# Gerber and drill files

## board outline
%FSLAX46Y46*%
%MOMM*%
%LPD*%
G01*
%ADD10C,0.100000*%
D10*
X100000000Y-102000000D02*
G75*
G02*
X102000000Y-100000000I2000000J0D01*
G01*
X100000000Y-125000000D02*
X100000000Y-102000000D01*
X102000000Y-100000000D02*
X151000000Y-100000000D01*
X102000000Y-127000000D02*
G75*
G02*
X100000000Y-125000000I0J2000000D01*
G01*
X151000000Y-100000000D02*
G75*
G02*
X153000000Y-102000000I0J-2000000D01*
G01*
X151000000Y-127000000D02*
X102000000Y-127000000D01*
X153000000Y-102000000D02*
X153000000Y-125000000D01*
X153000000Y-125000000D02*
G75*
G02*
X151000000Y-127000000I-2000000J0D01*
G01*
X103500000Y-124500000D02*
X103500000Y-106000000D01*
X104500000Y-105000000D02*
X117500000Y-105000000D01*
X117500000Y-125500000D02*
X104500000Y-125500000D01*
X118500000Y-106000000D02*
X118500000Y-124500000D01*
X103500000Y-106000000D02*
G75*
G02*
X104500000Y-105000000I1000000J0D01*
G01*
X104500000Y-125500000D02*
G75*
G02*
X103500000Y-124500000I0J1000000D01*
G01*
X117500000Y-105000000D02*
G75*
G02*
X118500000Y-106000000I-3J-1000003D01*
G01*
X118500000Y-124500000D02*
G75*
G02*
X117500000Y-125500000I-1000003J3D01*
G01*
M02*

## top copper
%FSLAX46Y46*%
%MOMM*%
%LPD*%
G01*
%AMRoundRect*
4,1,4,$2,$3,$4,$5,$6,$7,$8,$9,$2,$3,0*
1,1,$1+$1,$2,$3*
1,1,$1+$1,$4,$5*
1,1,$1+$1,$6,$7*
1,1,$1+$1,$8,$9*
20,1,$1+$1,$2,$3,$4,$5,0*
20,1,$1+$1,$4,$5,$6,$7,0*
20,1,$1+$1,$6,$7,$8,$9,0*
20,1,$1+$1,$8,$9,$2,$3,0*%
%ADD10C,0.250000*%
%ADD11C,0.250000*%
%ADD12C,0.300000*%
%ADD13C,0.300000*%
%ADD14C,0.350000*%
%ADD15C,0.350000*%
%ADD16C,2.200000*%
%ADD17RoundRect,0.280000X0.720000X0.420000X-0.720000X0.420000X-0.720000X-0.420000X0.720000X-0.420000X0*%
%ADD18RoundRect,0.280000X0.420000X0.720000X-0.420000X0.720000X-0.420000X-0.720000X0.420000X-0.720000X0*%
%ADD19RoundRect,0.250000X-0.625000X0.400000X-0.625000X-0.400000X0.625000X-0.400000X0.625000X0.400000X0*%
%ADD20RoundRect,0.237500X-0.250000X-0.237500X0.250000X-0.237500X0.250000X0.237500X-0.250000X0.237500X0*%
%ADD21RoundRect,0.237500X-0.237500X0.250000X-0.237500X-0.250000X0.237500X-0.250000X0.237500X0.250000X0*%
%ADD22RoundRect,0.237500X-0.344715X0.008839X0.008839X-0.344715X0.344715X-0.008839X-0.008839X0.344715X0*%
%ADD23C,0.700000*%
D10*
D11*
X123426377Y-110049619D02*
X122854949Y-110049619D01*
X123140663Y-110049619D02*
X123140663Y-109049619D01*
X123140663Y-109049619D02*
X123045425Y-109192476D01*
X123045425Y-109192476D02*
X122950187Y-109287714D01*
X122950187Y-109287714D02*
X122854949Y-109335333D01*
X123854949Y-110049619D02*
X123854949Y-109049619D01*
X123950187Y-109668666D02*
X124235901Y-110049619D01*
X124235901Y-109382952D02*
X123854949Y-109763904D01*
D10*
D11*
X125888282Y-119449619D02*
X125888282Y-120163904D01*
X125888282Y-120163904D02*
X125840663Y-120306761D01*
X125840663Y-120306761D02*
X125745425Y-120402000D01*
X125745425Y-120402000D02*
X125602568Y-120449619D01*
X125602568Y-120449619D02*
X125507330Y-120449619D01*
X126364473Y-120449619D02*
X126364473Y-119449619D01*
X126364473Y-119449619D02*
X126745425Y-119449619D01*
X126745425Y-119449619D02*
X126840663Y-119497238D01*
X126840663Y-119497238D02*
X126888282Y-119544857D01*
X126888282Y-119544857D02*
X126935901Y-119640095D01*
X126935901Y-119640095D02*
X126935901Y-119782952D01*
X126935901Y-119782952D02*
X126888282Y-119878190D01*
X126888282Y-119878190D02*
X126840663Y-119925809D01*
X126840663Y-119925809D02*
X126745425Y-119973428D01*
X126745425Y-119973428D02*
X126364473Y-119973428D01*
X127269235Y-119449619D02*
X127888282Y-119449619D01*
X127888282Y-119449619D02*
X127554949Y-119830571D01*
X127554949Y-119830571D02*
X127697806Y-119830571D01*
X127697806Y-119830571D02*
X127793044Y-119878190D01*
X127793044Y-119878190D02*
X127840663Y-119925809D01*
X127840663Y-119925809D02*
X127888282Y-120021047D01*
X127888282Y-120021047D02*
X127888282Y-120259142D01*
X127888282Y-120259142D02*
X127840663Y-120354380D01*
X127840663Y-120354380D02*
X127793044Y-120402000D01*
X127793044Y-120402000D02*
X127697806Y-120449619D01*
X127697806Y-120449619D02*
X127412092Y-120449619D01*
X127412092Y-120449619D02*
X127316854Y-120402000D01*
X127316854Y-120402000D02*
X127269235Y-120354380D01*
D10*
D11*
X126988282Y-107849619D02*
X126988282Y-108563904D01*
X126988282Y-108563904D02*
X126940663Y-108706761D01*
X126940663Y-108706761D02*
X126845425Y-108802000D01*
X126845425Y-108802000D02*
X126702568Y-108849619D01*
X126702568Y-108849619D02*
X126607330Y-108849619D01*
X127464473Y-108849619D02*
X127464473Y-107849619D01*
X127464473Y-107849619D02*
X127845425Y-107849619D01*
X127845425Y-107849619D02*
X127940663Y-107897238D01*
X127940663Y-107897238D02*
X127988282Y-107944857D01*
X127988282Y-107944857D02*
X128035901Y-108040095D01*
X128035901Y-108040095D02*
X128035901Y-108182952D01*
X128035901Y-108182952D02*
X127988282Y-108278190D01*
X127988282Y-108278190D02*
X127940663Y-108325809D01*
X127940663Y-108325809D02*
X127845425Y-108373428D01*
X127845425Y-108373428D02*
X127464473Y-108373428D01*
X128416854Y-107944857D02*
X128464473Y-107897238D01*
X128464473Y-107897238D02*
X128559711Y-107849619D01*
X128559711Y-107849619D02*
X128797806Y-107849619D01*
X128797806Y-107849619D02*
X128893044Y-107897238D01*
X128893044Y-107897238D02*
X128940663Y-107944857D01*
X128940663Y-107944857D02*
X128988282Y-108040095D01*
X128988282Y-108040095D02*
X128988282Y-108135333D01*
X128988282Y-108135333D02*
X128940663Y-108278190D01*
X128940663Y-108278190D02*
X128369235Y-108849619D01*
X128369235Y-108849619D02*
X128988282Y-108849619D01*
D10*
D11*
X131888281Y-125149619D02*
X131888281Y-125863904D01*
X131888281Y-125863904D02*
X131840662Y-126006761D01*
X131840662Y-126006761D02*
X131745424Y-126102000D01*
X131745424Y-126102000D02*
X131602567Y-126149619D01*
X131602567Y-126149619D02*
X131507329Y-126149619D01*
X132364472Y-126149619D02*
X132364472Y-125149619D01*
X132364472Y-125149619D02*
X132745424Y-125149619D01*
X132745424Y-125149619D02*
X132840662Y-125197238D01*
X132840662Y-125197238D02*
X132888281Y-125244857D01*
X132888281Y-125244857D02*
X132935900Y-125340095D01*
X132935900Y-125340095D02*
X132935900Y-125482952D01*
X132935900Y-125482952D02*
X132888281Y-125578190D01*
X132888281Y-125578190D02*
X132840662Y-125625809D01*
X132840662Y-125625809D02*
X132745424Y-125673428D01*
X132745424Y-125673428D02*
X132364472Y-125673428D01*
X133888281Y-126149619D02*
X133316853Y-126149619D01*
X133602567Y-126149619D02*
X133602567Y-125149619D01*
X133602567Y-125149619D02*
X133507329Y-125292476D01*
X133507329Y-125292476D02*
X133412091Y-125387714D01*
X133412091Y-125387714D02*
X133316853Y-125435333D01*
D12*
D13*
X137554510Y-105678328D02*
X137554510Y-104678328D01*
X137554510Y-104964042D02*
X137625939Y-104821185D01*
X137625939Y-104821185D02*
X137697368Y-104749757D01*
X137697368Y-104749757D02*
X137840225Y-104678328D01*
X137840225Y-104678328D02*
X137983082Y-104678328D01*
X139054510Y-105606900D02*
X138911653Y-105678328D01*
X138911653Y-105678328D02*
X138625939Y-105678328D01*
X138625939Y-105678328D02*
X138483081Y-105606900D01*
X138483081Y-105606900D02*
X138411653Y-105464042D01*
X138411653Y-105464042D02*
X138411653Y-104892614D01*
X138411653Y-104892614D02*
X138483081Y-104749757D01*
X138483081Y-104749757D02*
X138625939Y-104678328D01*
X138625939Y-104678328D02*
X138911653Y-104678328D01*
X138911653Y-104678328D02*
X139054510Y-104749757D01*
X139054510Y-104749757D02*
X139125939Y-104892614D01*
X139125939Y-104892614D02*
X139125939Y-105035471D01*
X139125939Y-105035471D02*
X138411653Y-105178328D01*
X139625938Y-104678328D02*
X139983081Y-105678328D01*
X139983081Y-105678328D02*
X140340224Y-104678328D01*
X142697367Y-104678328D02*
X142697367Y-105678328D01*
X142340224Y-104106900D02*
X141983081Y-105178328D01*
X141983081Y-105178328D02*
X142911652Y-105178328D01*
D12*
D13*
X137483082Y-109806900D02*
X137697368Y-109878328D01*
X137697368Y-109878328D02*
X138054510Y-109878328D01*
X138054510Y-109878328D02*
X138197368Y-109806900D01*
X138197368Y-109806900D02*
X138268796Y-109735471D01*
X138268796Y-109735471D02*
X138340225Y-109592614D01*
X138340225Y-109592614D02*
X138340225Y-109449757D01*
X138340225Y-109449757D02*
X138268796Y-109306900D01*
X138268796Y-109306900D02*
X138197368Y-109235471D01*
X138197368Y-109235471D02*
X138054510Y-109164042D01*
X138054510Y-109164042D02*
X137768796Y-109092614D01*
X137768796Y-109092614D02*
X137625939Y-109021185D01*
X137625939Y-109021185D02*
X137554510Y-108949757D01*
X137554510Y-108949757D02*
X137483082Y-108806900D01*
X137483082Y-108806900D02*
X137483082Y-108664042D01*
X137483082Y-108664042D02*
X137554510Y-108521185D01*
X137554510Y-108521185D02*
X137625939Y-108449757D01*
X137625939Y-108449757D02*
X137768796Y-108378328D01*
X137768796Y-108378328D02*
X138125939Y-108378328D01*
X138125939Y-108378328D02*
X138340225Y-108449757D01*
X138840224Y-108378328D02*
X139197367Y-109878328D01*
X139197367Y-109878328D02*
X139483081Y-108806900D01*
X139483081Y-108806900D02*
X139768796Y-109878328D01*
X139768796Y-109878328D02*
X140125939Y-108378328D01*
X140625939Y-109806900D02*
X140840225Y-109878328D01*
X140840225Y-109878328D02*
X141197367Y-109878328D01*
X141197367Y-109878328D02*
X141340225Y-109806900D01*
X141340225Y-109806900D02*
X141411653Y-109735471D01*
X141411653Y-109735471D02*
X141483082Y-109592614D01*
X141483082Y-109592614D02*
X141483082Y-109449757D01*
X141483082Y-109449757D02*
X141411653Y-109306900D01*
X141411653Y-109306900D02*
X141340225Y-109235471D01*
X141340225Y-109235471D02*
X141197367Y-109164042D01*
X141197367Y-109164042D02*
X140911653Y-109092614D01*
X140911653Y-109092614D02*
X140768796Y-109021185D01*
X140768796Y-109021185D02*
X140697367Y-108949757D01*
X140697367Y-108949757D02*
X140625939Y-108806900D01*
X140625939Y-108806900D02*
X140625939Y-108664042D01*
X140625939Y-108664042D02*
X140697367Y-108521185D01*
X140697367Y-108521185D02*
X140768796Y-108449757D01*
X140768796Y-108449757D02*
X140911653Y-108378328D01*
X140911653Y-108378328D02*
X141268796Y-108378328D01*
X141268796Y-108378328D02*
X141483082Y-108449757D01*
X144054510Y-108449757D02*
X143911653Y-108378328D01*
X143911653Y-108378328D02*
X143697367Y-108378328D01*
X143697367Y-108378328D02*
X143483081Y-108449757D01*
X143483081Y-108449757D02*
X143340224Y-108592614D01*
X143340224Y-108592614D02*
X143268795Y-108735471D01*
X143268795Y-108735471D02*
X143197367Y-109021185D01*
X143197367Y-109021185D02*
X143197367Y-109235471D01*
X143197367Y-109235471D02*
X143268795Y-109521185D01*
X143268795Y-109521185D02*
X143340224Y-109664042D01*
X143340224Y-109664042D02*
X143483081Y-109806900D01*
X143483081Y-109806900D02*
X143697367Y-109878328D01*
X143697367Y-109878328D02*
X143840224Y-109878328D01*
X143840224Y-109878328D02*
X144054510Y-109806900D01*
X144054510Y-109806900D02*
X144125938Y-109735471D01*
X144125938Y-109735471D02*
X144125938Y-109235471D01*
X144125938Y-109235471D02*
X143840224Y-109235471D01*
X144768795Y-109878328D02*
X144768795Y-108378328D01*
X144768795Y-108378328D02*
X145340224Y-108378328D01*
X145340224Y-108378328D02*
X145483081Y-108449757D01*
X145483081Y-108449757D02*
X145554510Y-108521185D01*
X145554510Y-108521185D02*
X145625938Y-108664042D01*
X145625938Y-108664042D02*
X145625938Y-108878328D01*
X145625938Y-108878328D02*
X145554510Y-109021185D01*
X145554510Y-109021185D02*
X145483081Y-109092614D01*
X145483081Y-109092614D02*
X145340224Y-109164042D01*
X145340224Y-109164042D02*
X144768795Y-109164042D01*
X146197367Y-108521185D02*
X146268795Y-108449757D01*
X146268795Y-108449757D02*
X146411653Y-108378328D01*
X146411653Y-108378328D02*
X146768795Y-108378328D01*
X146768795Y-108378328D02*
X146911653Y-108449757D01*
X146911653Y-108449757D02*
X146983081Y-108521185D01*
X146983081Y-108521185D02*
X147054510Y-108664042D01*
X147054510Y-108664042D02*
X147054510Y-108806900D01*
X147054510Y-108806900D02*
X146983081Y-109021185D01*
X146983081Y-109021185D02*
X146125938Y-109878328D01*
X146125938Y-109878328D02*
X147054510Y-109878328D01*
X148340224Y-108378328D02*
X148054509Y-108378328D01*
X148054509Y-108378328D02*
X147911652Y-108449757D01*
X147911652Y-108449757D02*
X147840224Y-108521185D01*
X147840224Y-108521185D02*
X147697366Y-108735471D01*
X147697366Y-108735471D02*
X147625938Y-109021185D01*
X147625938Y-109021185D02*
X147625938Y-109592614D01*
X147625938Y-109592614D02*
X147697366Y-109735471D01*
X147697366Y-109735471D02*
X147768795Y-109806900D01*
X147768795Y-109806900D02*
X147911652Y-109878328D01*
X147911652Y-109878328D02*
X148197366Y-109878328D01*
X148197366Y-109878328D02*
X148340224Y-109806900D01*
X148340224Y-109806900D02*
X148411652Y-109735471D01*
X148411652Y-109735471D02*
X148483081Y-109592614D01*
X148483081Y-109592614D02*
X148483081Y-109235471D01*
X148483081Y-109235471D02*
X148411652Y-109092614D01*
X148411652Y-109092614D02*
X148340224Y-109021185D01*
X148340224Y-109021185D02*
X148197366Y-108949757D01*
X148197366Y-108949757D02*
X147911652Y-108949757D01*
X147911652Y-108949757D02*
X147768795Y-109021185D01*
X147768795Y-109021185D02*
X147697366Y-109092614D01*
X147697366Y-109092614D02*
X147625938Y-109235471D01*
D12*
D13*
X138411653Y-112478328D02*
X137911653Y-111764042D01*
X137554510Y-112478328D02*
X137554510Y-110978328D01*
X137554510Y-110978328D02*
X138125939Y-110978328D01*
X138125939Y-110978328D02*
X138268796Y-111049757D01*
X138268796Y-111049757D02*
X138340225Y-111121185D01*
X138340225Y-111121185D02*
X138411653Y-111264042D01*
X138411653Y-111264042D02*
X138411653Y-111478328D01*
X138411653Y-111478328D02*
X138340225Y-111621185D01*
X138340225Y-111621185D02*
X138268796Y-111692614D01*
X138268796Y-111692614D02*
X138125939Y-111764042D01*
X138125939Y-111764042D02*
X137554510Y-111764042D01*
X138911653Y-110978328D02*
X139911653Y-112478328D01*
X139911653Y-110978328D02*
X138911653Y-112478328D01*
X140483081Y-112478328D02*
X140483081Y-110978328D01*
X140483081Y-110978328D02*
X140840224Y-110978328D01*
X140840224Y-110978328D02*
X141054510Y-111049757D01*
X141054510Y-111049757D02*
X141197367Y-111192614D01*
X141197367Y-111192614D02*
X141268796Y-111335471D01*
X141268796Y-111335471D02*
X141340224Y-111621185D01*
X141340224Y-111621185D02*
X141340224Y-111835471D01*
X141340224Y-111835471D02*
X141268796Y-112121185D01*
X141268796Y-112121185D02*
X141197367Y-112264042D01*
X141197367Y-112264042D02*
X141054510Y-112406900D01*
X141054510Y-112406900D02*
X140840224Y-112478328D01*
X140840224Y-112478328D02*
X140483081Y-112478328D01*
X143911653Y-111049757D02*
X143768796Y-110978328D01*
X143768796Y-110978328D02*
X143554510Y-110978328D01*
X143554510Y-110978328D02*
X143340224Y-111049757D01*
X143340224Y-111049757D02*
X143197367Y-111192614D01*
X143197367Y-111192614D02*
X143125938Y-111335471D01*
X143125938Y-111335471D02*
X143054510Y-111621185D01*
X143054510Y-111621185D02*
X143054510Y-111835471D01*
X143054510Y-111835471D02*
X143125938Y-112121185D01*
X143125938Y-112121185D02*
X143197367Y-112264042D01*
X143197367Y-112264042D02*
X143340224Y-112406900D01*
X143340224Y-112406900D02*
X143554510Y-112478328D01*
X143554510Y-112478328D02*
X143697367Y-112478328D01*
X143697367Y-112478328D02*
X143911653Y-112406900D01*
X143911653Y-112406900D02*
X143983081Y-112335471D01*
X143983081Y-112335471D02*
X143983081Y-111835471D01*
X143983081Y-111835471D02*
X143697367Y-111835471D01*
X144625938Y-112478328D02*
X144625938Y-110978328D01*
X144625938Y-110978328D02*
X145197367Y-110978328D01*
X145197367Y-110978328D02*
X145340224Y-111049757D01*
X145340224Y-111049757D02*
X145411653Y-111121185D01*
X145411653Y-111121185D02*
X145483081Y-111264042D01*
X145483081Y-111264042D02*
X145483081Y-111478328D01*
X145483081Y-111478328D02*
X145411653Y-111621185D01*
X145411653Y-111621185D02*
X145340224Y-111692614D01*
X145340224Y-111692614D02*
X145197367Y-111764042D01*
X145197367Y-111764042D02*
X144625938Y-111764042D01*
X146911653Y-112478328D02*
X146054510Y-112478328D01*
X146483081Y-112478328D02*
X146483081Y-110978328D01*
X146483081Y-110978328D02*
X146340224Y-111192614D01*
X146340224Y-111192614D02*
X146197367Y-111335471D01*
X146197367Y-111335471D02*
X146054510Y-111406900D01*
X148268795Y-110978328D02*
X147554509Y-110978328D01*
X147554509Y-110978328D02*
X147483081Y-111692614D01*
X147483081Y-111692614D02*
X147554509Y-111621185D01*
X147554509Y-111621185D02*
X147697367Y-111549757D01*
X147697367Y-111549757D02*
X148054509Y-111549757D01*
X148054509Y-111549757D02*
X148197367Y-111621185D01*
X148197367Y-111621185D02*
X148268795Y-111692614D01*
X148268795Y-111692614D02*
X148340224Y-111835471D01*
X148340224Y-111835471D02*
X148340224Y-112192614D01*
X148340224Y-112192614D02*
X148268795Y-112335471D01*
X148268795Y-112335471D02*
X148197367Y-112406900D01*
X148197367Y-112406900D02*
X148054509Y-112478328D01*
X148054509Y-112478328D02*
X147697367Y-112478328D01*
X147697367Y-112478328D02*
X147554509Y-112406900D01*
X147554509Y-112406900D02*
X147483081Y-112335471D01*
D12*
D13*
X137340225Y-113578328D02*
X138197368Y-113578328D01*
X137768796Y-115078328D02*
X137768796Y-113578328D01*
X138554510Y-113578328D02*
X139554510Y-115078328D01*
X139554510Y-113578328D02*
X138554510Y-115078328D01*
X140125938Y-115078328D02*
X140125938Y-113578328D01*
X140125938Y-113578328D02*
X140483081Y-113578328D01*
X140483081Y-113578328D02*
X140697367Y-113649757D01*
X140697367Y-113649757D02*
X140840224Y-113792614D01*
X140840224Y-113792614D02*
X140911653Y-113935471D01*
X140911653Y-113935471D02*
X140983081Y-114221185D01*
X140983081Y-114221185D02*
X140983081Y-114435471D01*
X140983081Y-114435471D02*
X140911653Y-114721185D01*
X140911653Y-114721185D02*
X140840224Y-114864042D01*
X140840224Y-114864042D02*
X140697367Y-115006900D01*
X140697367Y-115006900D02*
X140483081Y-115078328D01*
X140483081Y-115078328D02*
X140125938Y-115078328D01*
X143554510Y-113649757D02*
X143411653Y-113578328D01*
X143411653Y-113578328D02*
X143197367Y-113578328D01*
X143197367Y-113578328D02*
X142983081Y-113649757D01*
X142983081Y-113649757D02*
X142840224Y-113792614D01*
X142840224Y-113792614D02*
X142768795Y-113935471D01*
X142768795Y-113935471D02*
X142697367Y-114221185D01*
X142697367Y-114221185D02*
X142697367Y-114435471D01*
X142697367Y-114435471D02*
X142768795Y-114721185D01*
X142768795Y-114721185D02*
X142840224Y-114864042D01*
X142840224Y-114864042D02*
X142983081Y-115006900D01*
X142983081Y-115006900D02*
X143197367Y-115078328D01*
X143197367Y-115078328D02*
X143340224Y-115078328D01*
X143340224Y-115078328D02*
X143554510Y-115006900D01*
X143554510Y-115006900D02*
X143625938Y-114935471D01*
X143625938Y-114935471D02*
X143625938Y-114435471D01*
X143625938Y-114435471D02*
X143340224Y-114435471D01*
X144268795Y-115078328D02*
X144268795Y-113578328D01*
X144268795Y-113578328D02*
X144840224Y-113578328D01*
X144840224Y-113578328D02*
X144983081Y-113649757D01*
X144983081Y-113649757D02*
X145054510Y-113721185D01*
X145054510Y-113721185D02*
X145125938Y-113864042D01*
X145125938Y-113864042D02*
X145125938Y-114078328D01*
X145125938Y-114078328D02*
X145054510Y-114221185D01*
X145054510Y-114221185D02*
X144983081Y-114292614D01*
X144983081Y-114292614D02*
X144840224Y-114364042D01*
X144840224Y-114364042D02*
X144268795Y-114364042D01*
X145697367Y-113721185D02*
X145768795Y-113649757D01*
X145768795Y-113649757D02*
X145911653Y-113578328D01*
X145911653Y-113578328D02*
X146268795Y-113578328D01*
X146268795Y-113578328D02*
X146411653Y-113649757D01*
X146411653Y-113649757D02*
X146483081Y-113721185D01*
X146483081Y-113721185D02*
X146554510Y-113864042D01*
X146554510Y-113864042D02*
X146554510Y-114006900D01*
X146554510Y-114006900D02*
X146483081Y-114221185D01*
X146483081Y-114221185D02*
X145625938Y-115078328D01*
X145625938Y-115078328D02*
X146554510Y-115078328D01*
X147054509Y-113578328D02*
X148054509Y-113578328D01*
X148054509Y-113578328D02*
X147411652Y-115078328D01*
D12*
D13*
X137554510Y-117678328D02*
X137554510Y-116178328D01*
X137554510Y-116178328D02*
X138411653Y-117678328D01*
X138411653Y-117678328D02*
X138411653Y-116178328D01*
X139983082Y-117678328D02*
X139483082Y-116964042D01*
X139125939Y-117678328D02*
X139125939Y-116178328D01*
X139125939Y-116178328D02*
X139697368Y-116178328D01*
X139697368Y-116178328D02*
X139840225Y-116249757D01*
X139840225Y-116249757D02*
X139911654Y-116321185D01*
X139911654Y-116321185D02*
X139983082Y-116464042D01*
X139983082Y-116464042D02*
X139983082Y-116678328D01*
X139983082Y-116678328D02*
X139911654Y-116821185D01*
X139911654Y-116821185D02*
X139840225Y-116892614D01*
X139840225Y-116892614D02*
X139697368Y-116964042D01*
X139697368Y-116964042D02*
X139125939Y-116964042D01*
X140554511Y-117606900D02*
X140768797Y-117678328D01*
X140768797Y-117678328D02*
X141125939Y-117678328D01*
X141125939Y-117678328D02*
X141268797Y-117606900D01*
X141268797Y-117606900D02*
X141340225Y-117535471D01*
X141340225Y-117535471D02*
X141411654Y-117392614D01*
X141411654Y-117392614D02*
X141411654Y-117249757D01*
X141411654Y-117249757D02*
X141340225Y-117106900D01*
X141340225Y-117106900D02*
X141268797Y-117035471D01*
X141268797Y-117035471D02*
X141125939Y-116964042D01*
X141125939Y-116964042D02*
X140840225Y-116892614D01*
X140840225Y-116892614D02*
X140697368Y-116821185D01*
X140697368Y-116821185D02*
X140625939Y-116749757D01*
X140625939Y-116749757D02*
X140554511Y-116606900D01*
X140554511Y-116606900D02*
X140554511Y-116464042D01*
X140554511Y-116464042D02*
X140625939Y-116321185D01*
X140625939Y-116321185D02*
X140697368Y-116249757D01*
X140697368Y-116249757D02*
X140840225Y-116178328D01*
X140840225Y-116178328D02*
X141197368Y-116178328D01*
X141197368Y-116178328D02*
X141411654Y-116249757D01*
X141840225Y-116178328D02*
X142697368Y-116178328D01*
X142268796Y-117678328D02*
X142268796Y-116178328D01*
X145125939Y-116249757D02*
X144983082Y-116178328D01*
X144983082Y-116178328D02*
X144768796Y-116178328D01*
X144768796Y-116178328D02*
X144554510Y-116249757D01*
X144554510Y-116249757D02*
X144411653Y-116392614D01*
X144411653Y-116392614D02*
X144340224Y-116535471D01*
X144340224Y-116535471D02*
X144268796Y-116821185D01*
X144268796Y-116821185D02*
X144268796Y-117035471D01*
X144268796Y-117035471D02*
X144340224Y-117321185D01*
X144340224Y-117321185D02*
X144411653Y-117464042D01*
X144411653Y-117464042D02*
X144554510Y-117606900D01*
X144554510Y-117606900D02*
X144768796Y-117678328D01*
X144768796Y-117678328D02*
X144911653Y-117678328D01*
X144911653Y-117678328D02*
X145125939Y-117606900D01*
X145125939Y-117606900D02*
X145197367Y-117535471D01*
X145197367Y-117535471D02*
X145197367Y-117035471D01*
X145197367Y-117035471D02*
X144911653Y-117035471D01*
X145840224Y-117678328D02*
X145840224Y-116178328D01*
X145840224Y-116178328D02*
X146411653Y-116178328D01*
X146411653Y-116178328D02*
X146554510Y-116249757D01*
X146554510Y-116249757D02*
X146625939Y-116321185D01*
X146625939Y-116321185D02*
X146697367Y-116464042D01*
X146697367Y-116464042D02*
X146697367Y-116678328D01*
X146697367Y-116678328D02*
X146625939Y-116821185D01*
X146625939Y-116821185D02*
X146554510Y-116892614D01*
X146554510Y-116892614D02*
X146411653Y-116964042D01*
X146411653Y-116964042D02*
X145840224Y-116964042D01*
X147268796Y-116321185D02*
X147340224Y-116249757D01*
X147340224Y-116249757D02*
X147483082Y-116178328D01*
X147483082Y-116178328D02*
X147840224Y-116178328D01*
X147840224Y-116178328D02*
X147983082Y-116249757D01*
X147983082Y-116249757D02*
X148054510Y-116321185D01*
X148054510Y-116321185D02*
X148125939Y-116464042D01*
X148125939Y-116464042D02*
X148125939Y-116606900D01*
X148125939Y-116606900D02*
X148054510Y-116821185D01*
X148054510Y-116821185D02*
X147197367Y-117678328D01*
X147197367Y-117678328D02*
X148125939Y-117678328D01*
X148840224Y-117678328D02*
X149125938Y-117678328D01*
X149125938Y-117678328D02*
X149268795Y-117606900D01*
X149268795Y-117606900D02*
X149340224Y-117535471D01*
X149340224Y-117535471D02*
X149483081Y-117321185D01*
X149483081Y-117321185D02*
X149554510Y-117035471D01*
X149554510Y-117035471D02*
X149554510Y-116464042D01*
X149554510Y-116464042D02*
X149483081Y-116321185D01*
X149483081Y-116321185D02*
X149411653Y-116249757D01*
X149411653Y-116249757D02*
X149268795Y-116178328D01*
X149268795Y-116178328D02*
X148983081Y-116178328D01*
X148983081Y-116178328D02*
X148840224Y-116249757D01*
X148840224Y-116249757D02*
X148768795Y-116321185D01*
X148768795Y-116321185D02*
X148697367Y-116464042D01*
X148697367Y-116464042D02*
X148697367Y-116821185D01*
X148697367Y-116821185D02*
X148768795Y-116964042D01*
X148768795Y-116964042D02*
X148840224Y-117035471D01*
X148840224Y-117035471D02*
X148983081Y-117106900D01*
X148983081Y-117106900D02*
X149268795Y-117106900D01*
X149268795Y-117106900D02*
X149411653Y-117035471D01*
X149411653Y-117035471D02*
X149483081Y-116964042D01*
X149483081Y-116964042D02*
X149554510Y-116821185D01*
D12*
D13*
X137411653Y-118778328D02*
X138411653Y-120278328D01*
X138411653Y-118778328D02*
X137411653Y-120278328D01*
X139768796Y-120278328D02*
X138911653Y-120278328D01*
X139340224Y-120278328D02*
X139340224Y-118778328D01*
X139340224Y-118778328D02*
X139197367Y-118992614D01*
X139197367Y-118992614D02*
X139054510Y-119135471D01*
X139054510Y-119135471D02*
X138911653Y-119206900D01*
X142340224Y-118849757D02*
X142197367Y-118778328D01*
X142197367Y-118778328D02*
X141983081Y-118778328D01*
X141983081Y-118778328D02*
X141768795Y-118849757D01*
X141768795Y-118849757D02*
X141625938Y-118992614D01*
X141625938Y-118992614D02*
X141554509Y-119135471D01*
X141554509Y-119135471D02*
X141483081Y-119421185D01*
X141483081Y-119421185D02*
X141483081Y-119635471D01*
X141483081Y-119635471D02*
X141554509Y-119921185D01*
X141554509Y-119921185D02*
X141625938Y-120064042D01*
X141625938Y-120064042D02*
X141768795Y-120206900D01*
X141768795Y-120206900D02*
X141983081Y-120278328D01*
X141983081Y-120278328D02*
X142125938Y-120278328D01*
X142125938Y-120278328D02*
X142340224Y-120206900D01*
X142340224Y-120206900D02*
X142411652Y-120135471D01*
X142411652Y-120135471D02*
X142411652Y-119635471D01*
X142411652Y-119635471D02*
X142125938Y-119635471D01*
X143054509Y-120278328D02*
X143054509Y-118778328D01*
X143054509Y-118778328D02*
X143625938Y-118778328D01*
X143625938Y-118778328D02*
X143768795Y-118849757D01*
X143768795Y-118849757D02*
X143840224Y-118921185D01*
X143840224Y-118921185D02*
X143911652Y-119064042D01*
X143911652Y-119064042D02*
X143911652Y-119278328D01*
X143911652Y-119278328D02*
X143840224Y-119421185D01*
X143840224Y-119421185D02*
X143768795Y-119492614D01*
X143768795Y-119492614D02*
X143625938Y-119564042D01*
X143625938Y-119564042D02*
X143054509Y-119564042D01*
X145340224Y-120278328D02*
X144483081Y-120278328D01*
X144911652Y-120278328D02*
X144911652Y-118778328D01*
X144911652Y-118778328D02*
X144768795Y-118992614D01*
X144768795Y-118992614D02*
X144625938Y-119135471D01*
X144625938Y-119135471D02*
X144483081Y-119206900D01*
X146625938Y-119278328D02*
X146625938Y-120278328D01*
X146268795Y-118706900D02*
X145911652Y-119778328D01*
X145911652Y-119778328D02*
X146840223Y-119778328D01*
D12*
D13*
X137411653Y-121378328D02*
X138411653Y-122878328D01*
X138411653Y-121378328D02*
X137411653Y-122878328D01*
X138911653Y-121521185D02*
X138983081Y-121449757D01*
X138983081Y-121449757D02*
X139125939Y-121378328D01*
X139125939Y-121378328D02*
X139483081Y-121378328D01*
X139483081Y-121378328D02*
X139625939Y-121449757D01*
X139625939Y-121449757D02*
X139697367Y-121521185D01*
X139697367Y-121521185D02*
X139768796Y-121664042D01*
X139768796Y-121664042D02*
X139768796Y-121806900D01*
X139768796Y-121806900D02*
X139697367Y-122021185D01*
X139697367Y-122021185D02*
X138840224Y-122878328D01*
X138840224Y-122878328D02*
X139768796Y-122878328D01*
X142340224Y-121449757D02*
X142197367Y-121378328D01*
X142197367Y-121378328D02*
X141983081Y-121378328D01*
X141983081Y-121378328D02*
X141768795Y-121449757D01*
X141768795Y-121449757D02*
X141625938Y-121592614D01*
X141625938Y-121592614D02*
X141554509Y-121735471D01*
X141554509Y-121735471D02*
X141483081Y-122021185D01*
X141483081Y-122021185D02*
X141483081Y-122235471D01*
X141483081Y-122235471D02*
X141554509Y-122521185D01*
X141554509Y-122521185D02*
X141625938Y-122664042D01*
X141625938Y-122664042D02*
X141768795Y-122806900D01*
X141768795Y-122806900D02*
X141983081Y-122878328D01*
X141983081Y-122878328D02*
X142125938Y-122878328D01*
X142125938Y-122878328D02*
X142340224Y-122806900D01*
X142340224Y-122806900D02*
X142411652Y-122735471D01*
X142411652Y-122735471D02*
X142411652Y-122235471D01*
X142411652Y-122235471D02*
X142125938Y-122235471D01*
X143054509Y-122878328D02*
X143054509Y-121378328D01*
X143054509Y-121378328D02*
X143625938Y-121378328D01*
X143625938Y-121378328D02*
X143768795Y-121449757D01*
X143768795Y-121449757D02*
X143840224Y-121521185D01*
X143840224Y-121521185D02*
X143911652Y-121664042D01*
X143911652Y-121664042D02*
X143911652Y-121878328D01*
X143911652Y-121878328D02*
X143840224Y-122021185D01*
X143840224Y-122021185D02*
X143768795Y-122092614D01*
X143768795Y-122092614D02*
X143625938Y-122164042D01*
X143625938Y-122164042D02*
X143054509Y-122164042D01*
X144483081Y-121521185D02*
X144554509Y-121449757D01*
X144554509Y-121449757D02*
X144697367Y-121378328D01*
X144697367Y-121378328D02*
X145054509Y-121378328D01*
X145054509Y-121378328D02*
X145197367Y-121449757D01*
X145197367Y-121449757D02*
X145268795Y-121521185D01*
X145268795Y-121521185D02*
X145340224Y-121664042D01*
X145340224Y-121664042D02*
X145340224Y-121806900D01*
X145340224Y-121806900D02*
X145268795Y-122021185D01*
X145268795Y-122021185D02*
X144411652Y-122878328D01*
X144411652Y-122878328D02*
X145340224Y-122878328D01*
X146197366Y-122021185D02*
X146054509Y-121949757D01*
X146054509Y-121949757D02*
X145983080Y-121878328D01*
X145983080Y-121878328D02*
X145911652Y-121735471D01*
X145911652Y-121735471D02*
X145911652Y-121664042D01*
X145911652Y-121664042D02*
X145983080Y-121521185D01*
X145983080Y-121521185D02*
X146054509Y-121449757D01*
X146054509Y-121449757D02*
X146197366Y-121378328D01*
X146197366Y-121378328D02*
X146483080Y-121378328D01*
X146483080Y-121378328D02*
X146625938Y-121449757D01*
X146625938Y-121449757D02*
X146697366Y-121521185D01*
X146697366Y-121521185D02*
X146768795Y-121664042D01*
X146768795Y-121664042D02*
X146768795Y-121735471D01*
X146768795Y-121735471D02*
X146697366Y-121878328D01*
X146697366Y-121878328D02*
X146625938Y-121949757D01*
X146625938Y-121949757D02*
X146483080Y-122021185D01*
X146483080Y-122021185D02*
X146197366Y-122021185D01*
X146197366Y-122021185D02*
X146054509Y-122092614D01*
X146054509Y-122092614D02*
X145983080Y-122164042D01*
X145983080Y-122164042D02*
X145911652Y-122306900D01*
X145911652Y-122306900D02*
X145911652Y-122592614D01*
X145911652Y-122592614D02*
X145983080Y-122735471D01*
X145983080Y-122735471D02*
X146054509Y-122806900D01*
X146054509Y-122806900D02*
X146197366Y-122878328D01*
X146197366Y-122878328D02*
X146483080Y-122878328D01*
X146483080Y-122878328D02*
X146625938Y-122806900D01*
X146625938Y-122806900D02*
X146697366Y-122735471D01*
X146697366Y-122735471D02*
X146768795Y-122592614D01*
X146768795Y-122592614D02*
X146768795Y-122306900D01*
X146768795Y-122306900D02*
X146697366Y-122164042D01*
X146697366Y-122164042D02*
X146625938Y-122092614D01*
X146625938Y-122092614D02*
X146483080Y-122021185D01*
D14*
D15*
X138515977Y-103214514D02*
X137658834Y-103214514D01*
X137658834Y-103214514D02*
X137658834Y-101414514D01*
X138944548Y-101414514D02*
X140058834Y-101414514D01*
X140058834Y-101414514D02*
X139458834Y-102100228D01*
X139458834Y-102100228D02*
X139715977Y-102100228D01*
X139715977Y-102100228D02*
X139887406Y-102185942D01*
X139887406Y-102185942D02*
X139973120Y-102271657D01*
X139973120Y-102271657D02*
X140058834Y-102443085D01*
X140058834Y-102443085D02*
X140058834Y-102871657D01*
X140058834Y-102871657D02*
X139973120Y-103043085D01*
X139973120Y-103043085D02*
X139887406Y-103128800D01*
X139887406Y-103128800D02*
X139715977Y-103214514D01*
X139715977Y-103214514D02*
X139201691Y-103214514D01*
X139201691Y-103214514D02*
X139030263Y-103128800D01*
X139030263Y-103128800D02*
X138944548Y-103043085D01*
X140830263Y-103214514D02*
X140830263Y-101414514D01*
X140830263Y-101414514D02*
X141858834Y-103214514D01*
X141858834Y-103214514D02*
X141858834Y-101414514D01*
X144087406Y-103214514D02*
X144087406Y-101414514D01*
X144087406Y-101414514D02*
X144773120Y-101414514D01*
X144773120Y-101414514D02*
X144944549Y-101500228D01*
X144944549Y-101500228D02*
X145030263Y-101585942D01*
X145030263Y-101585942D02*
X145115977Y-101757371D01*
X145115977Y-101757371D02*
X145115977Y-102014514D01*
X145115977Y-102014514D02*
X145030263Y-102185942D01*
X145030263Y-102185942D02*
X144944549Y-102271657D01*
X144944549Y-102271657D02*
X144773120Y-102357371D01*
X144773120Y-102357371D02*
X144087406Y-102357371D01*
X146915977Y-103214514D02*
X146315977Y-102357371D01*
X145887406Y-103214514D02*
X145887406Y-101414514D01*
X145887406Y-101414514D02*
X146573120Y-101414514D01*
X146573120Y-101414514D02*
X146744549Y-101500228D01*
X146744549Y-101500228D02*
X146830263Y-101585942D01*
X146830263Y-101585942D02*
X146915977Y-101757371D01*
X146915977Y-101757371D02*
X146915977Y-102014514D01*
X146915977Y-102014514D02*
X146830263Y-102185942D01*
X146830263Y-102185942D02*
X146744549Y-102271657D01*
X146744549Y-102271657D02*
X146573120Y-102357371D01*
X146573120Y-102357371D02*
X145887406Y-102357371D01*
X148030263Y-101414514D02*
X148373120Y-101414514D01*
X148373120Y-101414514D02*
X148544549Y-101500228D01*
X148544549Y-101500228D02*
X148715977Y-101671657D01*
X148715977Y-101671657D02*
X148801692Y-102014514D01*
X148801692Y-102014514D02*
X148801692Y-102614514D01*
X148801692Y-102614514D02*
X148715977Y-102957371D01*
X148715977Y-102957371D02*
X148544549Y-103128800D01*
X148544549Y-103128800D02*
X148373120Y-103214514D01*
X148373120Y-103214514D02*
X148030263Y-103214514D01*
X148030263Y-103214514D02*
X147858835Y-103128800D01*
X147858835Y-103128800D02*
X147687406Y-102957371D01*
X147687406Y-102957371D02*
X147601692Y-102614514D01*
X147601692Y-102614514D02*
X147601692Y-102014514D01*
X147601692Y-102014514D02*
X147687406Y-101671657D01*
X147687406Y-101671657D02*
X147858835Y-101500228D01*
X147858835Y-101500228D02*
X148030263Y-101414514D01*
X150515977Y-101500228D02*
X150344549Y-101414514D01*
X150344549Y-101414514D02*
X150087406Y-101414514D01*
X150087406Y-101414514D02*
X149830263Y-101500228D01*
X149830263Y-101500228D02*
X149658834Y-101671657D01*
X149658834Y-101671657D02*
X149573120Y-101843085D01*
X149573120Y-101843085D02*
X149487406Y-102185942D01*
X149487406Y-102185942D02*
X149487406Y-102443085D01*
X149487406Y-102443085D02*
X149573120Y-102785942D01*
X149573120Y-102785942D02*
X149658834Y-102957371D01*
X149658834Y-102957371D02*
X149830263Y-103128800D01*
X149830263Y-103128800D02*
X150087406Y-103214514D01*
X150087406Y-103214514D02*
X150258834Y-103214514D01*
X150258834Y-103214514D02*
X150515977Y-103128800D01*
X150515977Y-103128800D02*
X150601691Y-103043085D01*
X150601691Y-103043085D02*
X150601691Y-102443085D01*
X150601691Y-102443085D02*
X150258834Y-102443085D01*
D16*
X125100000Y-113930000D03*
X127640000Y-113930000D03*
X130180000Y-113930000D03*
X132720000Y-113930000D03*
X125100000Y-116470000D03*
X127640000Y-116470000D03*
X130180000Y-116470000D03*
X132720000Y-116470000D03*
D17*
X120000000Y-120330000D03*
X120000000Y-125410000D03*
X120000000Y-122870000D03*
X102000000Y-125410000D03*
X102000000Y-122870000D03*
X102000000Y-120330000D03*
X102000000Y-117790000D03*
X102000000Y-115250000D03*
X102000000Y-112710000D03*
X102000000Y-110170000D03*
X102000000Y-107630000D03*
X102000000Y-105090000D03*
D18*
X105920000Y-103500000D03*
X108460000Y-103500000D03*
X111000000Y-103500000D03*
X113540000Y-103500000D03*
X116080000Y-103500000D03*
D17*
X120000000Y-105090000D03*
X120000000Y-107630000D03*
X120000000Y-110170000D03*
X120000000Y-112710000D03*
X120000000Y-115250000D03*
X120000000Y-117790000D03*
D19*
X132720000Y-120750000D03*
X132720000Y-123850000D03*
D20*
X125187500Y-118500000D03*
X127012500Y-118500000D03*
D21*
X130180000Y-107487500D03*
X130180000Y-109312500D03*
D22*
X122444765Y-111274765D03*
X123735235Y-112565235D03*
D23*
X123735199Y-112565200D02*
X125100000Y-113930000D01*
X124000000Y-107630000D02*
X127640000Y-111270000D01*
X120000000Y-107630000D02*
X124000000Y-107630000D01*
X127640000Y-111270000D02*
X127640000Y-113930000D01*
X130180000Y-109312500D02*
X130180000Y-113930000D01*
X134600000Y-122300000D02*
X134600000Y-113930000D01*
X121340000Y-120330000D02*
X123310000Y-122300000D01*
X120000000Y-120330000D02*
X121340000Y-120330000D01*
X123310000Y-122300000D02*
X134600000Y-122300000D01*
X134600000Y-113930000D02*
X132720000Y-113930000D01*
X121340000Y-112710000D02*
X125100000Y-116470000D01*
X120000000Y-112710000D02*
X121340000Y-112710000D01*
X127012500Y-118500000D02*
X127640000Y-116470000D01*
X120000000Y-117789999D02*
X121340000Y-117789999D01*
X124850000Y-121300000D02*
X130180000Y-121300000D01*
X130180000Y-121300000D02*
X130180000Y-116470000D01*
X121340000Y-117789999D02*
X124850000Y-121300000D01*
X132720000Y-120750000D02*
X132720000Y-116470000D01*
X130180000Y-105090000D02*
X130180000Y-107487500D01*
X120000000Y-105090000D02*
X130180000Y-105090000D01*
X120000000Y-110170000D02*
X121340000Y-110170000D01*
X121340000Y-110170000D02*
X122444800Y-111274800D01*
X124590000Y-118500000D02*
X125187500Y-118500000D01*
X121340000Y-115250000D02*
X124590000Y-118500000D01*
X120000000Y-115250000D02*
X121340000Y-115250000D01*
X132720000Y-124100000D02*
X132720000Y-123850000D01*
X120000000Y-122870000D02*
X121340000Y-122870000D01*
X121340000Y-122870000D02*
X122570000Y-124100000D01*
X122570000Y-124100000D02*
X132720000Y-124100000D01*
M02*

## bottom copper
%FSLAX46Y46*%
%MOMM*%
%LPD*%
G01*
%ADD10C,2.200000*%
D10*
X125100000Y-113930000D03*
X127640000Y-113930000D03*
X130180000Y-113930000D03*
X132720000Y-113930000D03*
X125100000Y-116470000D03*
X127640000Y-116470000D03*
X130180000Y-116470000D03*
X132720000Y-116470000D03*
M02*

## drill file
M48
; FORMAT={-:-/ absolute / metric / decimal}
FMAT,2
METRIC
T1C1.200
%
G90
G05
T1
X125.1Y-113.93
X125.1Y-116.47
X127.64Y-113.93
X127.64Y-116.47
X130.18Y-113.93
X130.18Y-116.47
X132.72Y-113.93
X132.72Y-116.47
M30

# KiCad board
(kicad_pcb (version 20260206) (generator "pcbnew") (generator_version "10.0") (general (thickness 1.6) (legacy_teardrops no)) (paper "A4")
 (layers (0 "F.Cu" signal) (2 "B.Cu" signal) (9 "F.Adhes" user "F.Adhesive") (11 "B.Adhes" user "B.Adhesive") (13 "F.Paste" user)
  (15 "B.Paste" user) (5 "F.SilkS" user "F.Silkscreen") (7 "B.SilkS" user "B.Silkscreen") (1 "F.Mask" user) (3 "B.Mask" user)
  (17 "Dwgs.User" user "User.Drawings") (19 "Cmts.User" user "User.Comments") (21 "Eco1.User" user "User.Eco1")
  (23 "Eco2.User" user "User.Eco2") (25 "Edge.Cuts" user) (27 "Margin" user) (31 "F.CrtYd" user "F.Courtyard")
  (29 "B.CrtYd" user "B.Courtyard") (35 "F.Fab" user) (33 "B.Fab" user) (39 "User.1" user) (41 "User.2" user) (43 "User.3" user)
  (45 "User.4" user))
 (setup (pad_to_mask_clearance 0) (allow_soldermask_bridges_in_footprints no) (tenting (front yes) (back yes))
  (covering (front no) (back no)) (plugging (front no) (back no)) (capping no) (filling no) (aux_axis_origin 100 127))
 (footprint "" (layer "F.Cu") (at 125.1 113.93)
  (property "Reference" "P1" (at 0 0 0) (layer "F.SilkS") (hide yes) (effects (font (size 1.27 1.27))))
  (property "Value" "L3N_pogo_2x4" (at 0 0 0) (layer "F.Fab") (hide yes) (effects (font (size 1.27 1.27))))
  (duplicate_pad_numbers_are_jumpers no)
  (pad "1" thru_hole circle (at 0 0) (size 2.2 2.2) (drill 1.2) (layers "F.Cu") (remove_unused_layers no) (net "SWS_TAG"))
  (pad "2" thru_hole circle (at 2.54 0) (size 2.2 2.2) (drill 1.2) (layers "F.Cu") (remove_unused_layers no) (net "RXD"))
  (pad "3" thru_hole circle (at 5.08 0) (size 2.2 2.2) (drill 1.2) (layers "F.Cu") (remove_unused_layers no) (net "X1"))
  (pad "4" thru_hole circle (at 7.62 0) (size 2.2 2.2) (drill 1.2) (layers "F.Cu") (remove_unused_layers no) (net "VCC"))
  (pad "5" thru_hole circle (at 0 2.54) (size 2.2 2.2) (drill 1.2) (layers "F.Cu") (remove_unused_layers no) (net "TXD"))
  (pad "6" thru_hole circle (at 2.54 2.54) (size 2.2 2.2) (drill 1.2) (layers "F.Cu") (remove_unused_layers no) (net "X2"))
  (pad "7" thru_hole circle (at 5.08 2.54) (size 2.2 2.2) (drill 1.2) (layers "F.Cu") (remove_unused_layers no) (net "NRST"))
  (pad "8" thru_hole circle (at 7.62 2.54) (size 2.2 2.2) (drill 1.2) (layers "F.Cu") (remove_unused_layers no) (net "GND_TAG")))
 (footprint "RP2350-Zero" (layer "F.Cu") (at 111 115.25 180)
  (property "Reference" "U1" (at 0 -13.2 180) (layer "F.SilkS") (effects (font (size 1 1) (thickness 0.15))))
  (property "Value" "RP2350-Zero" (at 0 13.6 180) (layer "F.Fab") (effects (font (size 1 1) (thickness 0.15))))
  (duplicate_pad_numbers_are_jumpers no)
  (fp_line (start 7.5 -9.25) (end 7.5 9.25) (stroke (width 0.1) (type default)) (layer "Edge.Cuts"))
  (fp_line (start 6.5 10.25) (end -6.5 10.25) (stroke (width 0.1) (type default)) (layer "Edge.Cuts"))
  (fp_line (start -6.5 -10.25) (end 6.5 -10.25) (stroke (width 0.1) (type default)) (layer "Edge.Cuts"))
  (fp_line (start -7.5 9.25) (end -7.5 -9.25) (stroke (width 0.1) (type default)) (layer "Edge.Cuts"))
  (fp_arc (start 7.5 9.25) (mid 7.207106 9.957106) (end 6.5 10.25) (stroke (width 0.1) (type default)) (layer "Edge.Cuts"))
  (fp_arc (start 6.5 -10.25) (mid 7.207106 -9.957106) (end 7.5 -9.25) (stroke (width 0.1) (type default)) (layer "Edge.Cuts"))
  (fp_arc (start -6.5 10.25) (mid -7.207106 9.957106) (end -7.5 9.25) (stroke (width 0.1) (type default)) (layer "Edge.Cuts"))
  (fp_arc (start -7.5 -9.25) (mid -7.207106 -9.957106) (end -6.5 -10.25) (stroke (width 0.1) (type default)) (layer "Edge.Cuts"))
  (pad "3V3" smd roundrect (at -9 -5.08 180) (size 2 1.4) (layers "F.Cu" "F.Mask" "F.Paste") (roundrect_rratio 0.2) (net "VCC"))
  (pad "5V" smd roundrect (at -9 -10.16 180) (size 2 1.4) (layers "F.Cu" "F.Mask" "F.Paste") (roundrect_rratio 0.2))
  (pad "GND" smd roundrect (at -9 -7.62 180) (size 2 1.4) (layers "F.Cu" "F.Mask" "F.Paste") (roundrect_rratio 0.2) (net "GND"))
  (pad "GP0" smd roundrect (at 9 -10.16 180) (size 2 1.4) (layers "F.Cu" "F.Mask" "F.Paste") (roundrect_rratio 0.2))
  (pad "GP1" smd roundrect (at 9 -7.62 180) (size 2 1.4) (layers "F.Cu" "F.Mask" "F.Paste") (roundrect_rratio 0.2))
  (pad "GP2" smd roundrect (at 9 -5.08 180) (size 2 1.4) (layers "F.Cu" "F.Mask" "F.Paste") (roundrect_rratio 0.2))
  (pad "GP3" smd roundrect (at 9 -2.54 180) (size 2 1.4) (layers "F.Cu" "F.Mask" "F.Paste") (roundrect_rratio 0.2))
  (pad "GP4" smd roundrect (at 9 0 180) (size 2 1.4) (layers "F.Cu" "F.Mask" "F.Paste") (roundrect_rratio 0.2))
  (pad "GP5" smd roundrect (at 9 2.54 180) (size 2 1.4) (layers "F.Cu" "F.Mask" "F.Paste") (roundrect_rratio 0.2))
  (pad "GP6" smd roundrect (at 9 5.08 180) (size 2 1.4) (layers "F.Cu" "F.Mask" "F.Paste") (roundrect_rratio 0.2))
  (pad "GP7" smd roundrect (at 9 7.62 180) (size 2 1.4) (layers "F.Cu" "F.Mask" "F.Paste") (roundrect_rratio 0.2))
  (pad "GP8" smd roundrect (at 9 10.16 180) (size 2 1.4) (layers "F.Cu" "F.Mask" "F.Paste") (roundrect_rratio 0.2))
  (pad "GP9" smd roundrect (at 5.08 11.75 180) (size 1.4 2) (layers "F.Cu" "F.Mask" "F.Paste") (roundrect_rratio 0.2))
  (pad "GP10" smd roundrect (at 2.54 11.75 180) (size 1.4 2) (layers "F.Cu" "F.Mask" "F.Paste") (roundrect_rratio 0.2))
  (pad "GP11" smd roundrect (at 0 11.75 180) (size 1.4 2) (layers "F.Cu" "F.Mask" "F.Paste") (roundrect_rratio 0.2))
  (pad "GP12" smd roundrect (at -2.54 11.75 180) (size 1.4 2) (layers "F.Cu" "F.Mask" "F.Paste") (roundrect_rratio 0.2))
  (pad "GP13" smd roundrect (at -5.08 11.75 180) (size 1.4 2) (layers "F.Cu" "F.Mask" "F.Paste") (roundrect_rratio 0.2))
  (pad "GP14" smd roundrect (at -9 10.16 180) (size 2 1.4) (layers "F.Cu" "F.Mask" "F.Paste") (roundrect_rratio 0.2) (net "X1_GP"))
  (pad "GP15" smd roundrect (at -9 7.62 180) (size 2 1.4) (layers "F.Cu" "F.Mask" "F.Paste") (roundrect_rratio 0.2) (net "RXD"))
  (pad "GP26" smd roundrect (at -9 5.08 180) (size 2 1.4) (layers "F.Cu" "F.Mask" "F.Paste") (roundrect_rratio 0.2) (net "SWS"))
  (pad "GP27" smd roundrect (at -9 2.54 180) (size 2 1.4) (layers "F.Cu" "F.Mask" "F.Paste") (roundrect_rratio 0.2) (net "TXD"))
  (pad "GP28" smd roundrect (at -9 0 180) (size 2 1.4) (layers "F.Cu" "F.Mask" "F.Paste") (roundrect_rratio 0.2) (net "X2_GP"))
  (pad "GP29" smd roundrect (at -9 -2.54 180) (size 2 1.4) (layers "F.Cu" "F.Mask" "F.Paste") (roundrect_rratio 0.2) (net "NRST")))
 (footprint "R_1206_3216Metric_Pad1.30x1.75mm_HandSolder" (layer "F.Cu") (at 132.72 122.3 -90)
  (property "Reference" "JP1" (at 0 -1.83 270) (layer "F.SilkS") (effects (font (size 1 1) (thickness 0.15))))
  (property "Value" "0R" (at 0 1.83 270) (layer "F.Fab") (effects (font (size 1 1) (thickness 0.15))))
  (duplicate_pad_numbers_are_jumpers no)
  (pad "1" smd roundrect (at -1.55 0 270) (size 1.3 1.75) (layers "F.Cu" "F.Mask" "F.Paste") (roundrect_rratio 0.192308) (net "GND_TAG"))
  (pad "2" smd roundrect (at 1.55 0 270) (size 1.3 1.75) (layers "F.Cu" "F.Mask" "F.Paste") (roundrect_rratio 0.192308) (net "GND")))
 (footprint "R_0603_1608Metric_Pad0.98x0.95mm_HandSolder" (layer "F.Cu") (at 126.1 118.5)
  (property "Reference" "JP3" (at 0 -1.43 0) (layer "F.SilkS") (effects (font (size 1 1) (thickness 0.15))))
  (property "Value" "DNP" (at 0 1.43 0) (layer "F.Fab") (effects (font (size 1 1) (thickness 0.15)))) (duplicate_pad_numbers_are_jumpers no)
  (pad "1" smd roundrect (at -0.9125 0) (size 0.975 0.95) (layers "F.Cu" "F.Mask" "F.Paste") (roundrect_rratio 0.25) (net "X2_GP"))
  (pad "2" smd roundrect (at 0.9125 0) (size 0.975 0.95) (layers "F.Cu" "F.Mask" "F.Paste") (roundrect_rratio 0.25) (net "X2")))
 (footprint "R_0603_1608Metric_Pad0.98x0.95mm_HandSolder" (layer "F.Cu") (at 130.18 108.4 -90)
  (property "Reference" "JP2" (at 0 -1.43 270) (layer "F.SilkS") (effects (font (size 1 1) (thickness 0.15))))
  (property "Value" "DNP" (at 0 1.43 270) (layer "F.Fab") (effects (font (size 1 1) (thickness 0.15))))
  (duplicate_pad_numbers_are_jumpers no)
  (pad "1" smd roundrect (at -0.9125 0 270) (size 0.975 0.95) (layers "F.Cu" "F.Mask" "F.Paste") (roundrect_rratio 0.25) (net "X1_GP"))
  (pad "2" smd roundrect (at 0.9125 0 270) (size 0.975 0.95) (layers "F.Cu" "F.Mask" "F.Paste") (roundrect_rratio 0.25) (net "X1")))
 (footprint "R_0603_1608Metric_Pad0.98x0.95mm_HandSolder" (layer "F.Cu") (at 123.09 111.92 -45)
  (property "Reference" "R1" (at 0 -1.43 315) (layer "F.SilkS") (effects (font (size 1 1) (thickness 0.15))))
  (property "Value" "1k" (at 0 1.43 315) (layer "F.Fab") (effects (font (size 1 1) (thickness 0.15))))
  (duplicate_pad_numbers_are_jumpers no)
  (pad "1" smd roundrect (at -0.9125 0 315) (size 0.975 0.95) (layers "F.Cu" "F.Mask" "F.Paste") (roundrect_rratio 0.25) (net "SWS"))
  (pad "2" smd roundrect (at 0.9125 0 315) (size 0.975 0.95) (layers "F.Cu" "F.Mask" "F.Paste") (roundrect_rratio 0.25) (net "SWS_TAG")))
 (gr_arc (start 100 102) (mid 100.585786 100.585786) (end 102 100) (stroke (width 0.1) (type default)) (layer "Edge.Cuts"))
 (gr_line (start 100 125) (end 100 102) (stroke (width 0.1) (type default)) (layer "Edge.Cuts"))
 (gr_line (start 102 100) (end 151 100) (stroke (width 0.1) (type default)) (layer "Edge.Cuts"))
 (gr_arc (start 102 127) (mid 100.585786 126.414213) (end 100 125) (stroke (width 0.1) (type default)) (layer "Edge.Cuts"))
 (gr_arc (start 151 100) (mid 152.414213 100.585786) (end 153 102) (stroke (width 0.1) (type default)) (layer "Edge.Cuts"))
 (gr_line (start 151 127) (end 102 127) (stroke (width 0.1) (type default)) (layer "Edge.Cuts"))
 (gr_line (start 153 102) (end 153 125) (stroke (width 0.1) (type default)) (layer "Edge.Cuts"))
 (gr_arc (start 153 125) (mid 152.414213 126.414213) (end 151 127) (stroke (width 0.1) (type default)) (layer "Edge.Cuts"))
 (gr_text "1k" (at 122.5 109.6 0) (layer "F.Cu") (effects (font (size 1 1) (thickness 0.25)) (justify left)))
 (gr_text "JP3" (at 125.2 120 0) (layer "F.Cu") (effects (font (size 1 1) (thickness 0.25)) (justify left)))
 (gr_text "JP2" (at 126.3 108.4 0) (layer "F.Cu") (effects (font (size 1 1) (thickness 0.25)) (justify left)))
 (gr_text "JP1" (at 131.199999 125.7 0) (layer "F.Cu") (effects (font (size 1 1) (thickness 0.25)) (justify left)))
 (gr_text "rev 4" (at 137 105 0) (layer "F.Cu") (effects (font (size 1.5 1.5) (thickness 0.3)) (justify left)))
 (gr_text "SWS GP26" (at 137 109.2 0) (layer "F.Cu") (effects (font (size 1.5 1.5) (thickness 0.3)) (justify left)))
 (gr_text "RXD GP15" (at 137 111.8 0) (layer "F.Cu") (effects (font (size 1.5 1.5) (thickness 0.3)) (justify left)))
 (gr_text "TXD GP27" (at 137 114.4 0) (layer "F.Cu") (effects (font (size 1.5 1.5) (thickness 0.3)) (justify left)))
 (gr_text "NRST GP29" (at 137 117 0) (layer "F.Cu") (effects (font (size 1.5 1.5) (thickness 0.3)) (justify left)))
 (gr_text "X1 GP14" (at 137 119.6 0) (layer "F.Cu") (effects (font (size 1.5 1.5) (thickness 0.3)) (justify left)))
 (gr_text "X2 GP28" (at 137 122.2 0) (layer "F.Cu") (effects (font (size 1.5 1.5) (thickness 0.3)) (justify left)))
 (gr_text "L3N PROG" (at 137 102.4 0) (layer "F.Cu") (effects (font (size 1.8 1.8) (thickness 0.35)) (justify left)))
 (segment (start 123.735199 112.5652) (end 125.1 113.93) (width 0.7) (layer "F.Cu") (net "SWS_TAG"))
 (segment (start 124 107.63) (end 127.64 111.27) (width 0.7) (layer "F.Cu") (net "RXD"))
 (segment (start 120 107.63) (end 124 107.63) (width 0.7) (layer "F.Cu") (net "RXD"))
 (segment (start 127.64 111.27) (end 127.64 113.93) (width 0.7) (layer "F.Cu") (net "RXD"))
 (segment (start 130.18 109.3125) (end 130.18 113.93) (width 0.7) (layer "F.Cu") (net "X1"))
 (segment (start 134.6 122.3) (end 134.6 113.93) (width 0.7) (layer "F.Cu") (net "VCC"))
 (segment (start 121.34 120.33) (end 123.31 122.3) (width 0.7) (layer "F.Cu") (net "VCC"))
 (segment (start 120 120.33) (end 121.34 120.33) (width 0.7) (layer "F.Cu") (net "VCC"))
 (segment (start 123.31 122.3) (end 134.6 122.3) (width 0.7) (layer "F.Cu") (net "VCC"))
 (segment (start 134.6 113.93) (end 132.72 113.93) (width 0.7) (layer "F.Cu") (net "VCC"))
 (segment (start 121.34 112.71) (end 125.1 116.47) (width 0.7) (layer "F.Cu") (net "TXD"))
 (segment (start 120 112.71) (end 121.34 112.71) (width 0.7) (layer "F.Cu") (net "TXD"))
 (segment (start 127.0125 118.5) (end 127.64 116.47) (width 0.7) (layer "F.Cu") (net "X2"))
 (segment (start 120 117.789999) (end 121.34 117.789999) (width 0.7) (layer "F.Cu") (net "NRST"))
 (segment (start 124.85 121.3) (end 130.18 121.3) (width 0.7) (layer "F.Cu") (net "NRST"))
 (segment (start 130.18 121.3) (end 130.18 116.47) (width 0.7) (layer "F.Cu") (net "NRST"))
 (segment (start 121.34 117.789999) (end 124.85 121.3) (width 0.7) (layer "F.Cu") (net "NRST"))
 (segment (start 132.72 120.75) (end 132.72 116.47) (width 0.7) (layer "F.Cu") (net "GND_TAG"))
 (segment (start 130.18 105.09) (end 130.18 107.4875) (width 0.7) (layer "F.Cu") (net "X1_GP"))
 (segment (start 120 105.09) (end 130.18 105.09) (width 0.7) (layer "F.Cu") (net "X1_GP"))
 (segment (start 120 110.17) (end 121.34 110.17) (width 0.7) (layer "F.Cu") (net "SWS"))
 (segment (start 121.34 110.17) (end 122.4448 111.2748) (width 0.7) (layer "F.Cu") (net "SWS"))
 (segment (start 124.59 118.5) (end 125.1875 118.5) (width 0.7) (layer "F.Cu") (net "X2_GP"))
 (segment (start 121.34 115.25) (end 124.59 118.5) (width 0.7) (layer "F.Cu") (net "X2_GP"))
 (segment (start 120 115.25) (end 121.34 115.25) (width 0.7) (layer "F.Cu") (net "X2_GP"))
 (segment (start 132.72 124.1) (end 132.72 123.85) (width 0.7) (layer "F.Cu") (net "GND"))
 (segment (start 120 122.87) (end 121.34 122.87) (width 0.7) (layer "F.Cu") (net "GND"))
 (segment (start 121.34 122.87) (end 122.57 124.1) (width 0.7) (layer "F.Cu") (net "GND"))
 (segment (start 122.57 124.1) (end 132.72 124.1) (width 0.7) (layer "F.Cu") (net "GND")))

